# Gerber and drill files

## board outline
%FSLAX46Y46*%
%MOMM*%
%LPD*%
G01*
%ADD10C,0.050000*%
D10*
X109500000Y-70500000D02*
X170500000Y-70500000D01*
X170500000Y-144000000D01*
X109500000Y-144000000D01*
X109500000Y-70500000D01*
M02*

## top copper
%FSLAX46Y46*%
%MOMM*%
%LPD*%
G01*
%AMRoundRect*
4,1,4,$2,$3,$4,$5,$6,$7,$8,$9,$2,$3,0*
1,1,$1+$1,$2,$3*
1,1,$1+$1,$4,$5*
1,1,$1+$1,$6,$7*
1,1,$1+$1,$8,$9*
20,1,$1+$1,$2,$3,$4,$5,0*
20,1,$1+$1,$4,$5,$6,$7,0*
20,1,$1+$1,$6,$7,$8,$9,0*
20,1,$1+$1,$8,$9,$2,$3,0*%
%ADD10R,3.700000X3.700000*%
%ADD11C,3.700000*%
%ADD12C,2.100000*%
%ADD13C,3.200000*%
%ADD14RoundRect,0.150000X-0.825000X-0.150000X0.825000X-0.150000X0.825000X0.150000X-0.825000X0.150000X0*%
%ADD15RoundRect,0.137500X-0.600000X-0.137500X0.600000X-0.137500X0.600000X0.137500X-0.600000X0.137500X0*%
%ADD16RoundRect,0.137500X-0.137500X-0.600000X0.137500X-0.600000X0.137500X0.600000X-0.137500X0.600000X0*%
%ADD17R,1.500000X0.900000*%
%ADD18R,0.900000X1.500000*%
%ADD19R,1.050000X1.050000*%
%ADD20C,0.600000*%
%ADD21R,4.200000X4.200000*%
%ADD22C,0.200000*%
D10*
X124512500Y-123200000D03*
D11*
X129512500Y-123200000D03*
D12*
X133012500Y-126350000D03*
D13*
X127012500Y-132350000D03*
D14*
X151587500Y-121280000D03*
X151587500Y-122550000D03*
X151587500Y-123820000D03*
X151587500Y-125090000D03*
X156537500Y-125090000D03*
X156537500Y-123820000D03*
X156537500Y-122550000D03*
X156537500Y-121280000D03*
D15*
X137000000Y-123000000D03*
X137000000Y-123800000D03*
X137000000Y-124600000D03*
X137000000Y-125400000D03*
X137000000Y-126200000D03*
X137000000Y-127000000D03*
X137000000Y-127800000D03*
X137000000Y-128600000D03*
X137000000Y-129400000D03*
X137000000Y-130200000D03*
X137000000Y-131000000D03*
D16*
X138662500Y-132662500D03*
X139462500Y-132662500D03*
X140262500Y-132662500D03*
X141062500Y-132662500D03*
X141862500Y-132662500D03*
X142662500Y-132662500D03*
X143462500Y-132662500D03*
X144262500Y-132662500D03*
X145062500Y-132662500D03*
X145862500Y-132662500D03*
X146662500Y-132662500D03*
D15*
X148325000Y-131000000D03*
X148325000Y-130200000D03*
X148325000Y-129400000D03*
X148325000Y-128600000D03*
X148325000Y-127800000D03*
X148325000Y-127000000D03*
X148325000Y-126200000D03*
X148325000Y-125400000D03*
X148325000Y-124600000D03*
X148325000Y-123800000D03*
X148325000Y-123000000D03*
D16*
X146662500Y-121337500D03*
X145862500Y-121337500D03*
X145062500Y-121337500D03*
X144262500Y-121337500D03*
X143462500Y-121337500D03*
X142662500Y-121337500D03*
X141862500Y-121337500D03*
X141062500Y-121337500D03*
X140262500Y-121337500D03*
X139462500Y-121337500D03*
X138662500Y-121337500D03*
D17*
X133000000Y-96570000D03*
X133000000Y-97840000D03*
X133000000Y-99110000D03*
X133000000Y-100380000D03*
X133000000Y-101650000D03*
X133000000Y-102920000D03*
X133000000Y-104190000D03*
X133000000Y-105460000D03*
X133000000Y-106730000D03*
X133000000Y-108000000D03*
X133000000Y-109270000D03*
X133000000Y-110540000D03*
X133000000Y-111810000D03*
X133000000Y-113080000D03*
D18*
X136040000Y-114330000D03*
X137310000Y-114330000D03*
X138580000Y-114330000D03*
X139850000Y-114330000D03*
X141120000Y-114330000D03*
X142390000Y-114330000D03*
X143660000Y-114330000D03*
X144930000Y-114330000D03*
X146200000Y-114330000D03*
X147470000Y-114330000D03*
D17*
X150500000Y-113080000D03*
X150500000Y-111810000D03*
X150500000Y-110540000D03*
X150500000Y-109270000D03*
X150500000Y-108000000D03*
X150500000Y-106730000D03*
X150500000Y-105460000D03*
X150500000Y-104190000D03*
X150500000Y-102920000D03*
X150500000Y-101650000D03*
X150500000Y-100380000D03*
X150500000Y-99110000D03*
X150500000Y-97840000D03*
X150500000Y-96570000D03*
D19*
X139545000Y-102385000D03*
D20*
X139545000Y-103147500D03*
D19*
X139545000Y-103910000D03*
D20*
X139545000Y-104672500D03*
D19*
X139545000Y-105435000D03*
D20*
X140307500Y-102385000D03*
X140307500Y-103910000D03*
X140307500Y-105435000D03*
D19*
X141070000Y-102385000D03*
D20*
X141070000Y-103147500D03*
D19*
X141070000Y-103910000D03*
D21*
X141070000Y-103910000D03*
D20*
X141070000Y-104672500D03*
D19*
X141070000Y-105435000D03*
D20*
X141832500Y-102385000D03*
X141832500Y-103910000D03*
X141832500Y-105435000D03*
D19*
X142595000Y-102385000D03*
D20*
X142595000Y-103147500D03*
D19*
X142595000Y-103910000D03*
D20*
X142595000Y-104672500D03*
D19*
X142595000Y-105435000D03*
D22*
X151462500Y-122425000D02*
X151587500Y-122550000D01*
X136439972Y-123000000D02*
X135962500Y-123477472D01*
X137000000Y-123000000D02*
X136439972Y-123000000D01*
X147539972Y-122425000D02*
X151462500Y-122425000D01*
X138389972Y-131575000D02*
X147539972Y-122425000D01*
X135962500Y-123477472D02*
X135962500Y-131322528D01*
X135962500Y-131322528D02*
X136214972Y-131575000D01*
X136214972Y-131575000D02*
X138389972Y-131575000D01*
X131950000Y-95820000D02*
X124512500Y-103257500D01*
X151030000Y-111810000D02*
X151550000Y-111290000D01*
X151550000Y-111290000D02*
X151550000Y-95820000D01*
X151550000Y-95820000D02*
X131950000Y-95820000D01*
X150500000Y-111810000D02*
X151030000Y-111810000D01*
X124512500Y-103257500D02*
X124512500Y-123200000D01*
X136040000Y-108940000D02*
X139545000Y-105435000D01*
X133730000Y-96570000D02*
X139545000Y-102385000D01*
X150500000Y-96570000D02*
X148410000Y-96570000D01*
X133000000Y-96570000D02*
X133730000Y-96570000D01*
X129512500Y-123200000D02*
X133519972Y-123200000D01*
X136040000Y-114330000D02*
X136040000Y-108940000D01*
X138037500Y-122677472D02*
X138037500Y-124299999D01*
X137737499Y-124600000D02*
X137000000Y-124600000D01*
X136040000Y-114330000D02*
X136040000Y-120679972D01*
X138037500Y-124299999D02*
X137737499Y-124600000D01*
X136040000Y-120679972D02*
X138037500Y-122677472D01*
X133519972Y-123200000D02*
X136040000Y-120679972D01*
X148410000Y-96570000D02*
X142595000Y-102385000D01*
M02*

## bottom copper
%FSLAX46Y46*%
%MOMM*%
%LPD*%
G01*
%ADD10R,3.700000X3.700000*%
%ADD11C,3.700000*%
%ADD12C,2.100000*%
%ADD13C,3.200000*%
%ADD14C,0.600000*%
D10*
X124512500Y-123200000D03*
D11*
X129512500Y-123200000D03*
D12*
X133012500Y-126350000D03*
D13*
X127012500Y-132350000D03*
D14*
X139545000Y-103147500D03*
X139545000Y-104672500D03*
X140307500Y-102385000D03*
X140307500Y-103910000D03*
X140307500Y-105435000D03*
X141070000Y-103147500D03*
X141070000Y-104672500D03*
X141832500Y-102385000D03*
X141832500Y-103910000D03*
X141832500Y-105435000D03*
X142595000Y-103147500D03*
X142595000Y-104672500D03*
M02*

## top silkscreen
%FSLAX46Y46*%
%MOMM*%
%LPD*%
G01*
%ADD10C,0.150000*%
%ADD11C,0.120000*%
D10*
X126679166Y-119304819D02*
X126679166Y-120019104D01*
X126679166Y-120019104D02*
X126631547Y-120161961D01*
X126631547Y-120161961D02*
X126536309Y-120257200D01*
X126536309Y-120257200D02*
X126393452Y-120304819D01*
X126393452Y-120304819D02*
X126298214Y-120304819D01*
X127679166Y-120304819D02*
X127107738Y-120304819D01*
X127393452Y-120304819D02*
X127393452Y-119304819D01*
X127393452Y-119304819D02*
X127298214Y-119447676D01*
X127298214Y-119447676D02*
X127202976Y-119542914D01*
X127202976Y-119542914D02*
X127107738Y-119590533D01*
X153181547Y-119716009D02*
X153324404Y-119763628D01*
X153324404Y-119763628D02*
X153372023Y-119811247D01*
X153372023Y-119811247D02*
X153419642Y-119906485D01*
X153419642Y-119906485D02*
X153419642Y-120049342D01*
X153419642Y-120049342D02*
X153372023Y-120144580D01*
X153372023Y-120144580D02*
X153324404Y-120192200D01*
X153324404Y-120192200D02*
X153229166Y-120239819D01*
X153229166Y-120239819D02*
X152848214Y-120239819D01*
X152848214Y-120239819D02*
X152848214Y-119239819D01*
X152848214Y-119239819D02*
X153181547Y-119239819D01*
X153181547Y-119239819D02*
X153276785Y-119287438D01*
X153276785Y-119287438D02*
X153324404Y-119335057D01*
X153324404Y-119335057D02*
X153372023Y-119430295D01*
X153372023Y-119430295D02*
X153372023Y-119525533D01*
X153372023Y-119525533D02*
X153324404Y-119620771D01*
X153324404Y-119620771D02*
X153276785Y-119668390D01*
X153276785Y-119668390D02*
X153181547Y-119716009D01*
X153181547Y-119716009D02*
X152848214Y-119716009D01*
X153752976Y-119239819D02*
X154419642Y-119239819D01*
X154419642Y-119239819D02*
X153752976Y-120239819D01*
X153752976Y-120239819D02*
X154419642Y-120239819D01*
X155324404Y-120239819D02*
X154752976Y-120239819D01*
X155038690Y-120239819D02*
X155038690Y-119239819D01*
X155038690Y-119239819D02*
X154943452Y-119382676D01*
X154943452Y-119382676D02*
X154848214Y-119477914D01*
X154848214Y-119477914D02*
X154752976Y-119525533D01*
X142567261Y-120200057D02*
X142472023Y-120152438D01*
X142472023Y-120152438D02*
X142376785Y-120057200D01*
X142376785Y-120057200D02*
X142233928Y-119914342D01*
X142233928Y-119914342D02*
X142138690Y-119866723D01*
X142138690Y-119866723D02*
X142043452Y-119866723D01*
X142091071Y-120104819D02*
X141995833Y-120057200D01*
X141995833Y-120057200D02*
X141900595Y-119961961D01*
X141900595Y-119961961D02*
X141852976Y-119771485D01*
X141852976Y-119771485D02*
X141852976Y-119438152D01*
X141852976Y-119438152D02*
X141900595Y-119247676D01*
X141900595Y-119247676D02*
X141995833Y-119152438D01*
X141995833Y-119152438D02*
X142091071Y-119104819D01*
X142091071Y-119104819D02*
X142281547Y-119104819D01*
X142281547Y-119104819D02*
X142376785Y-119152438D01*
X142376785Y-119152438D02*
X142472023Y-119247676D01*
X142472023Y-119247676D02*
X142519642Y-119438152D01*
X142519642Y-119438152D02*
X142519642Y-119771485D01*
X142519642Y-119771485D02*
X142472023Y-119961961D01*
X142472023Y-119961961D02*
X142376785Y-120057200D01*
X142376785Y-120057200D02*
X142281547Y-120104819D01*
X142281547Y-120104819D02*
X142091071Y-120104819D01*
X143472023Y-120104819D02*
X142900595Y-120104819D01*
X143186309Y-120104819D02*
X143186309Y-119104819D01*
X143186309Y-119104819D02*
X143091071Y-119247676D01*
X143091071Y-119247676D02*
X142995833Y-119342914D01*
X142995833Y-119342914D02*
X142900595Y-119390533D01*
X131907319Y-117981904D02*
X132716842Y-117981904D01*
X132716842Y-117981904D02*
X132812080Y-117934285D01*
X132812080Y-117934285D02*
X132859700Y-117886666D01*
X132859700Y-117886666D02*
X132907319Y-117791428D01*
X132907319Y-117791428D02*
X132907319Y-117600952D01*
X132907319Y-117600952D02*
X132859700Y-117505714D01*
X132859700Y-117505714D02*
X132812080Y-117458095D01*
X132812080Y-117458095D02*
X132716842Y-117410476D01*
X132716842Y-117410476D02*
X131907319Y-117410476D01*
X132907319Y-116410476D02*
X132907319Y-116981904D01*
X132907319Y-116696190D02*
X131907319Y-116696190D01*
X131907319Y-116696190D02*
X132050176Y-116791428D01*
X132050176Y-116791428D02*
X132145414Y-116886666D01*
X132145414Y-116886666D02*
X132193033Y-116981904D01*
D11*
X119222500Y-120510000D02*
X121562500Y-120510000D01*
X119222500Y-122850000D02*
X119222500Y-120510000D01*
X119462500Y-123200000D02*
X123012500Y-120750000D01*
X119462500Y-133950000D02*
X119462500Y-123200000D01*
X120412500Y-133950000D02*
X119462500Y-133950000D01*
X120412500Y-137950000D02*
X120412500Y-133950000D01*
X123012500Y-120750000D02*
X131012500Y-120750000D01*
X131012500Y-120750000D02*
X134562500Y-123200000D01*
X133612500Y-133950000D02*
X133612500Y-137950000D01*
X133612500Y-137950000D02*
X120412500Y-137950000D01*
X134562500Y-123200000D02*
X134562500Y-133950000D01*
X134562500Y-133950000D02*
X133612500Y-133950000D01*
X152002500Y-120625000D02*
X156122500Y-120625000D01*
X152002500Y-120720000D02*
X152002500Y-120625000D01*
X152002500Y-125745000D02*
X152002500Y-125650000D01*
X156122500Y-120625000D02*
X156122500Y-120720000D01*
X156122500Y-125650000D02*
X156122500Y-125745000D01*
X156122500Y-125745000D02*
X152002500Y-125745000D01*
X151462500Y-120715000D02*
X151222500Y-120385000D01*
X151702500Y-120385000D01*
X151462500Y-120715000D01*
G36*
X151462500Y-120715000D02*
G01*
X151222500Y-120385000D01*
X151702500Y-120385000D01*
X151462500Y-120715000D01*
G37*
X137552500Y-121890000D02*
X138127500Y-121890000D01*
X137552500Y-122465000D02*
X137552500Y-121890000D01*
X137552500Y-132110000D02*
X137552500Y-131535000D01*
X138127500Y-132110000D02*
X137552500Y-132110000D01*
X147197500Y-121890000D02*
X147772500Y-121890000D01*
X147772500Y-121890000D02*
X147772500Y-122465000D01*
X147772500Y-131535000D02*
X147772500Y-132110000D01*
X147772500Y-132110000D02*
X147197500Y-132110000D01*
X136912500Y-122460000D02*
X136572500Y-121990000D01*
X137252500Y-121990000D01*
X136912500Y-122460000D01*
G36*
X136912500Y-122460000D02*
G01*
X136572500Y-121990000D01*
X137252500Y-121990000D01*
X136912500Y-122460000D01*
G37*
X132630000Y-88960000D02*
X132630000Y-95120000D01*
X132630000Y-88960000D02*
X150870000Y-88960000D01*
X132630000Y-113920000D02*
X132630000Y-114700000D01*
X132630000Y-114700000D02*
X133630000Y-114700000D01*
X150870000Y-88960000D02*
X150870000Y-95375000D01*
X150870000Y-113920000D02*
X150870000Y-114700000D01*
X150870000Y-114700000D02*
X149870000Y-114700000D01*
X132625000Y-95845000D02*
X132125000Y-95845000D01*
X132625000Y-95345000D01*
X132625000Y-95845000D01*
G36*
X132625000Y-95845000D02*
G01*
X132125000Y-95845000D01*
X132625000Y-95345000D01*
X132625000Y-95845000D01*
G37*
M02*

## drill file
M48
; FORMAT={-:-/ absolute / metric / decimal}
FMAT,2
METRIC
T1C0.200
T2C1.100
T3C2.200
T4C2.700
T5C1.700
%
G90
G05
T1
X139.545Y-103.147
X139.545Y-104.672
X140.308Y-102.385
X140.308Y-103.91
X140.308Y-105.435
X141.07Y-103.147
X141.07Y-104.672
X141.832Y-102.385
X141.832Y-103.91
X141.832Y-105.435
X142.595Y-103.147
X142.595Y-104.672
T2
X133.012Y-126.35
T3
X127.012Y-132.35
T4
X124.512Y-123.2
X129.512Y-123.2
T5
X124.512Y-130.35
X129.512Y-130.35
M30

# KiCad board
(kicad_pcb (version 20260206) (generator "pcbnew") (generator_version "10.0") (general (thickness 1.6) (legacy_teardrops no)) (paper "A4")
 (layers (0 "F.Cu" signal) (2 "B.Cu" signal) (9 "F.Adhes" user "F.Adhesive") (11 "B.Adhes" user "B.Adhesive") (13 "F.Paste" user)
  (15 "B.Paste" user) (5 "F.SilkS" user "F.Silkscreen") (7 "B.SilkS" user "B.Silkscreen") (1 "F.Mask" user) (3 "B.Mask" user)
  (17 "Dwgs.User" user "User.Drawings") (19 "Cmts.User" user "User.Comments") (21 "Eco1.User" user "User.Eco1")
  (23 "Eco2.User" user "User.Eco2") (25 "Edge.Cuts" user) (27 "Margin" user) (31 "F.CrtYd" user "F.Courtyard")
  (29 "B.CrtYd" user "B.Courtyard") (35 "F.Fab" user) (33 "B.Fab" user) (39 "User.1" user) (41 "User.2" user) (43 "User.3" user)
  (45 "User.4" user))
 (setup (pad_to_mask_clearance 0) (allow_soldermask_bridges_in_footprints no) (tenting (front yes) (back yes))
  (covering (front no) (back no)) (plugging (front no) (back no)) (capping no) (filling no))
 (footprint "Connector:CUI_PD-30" (layer "F.Cu") (at 124.5125 123.2)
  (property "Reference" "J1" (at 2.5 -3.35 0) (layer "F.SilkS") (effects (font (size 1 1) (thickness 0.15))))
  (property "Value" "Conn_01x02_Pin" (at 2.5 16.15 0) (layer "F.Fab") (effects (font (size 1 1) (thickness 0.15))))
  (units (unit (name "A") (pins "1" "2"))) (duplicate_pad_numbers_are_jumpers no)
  (fp_line (start -5.29 -2.69) (end -2.95 -2.69) (stroke (width 0.12) (type solid)) (layer "F.SilkS"))
  (fp_line (start -5.29 -0.35) (end -5.29 -2.69) (stroke (width 0.12) (type solid)) (layer "F.SilkS"))
  (fp_line (start -5.05 0) (end -1.5 -2.45) (stroke (width 0.12) (type solid)) (layer "F.SilkS"))
  (fp_line (start -5.05 10.75) (end -5.05 0) (stroke (width 0.12) (type solid)) (layer "F.SilkS"))
  (fp_line (start -4.1 10.75) (end -5.05 10.75) (stroke (width 0.12) (type solid)) (layer "F.SilkS"))
  (fp_line (start -4.1 14.75) (end -4.1 10.75) (stroke (width 0.12) (type solid)) (layer "F.SilkS"))
  (fp_line (start -1.5 -2.45) (end 6.5 -2.45) (stroke (width 0.12) (type solid)) (layer "F.SilkS"))
  (fp_line (start 6.5 -2.45) (end 10.05 0) (stroke (width 0.12) (type solid)) (layer "F.SilkS"))
  (fp_line (start 9.1 10.75) (end 9.1 14.75) (stroke (width 0.12) (type solid)) (layer "F.SilkS"))
  (fp_line (start 9.1 14.75) (end -4.1 14.75) (stroke (width 0.12) (type solid)) (layer "F.SilkS"))
  (fp_line (start 10.05 0) (end 10.05 10.75) (stroke (width 0.12) (type solid)) (layer "F.SilkS"))
  (fp_line (start 10.05 10.75) (end 9.1 10.75) (stroke (width 0.12) (type solid)) (layer "F.SilkS"))
  (pad "" np_thru_hole circle (at 0 7.15 180) (size 1.7 1.7) (drill 1.7) (layers "*.Cu" "*.Mask"))
  (pad "" np_thru_hole circle (at 5 7.15 180) (size 1.7 1.7) (drill 1.7) (layers "*.Cu" "*.Mask"))
  (pad "1" thru_hole rect (at 0 0 180) (size 3.7 3.7) (drill 2.7) (layers "*.Cu" "*.Mask") (remove_unused_layers no) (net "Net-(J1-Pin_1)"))
  (pad "2" thru_hole circle (at 5 0 180) (size 3.7 3.7) (drill 2.7) (layers "*.Cu" "*.Mask") (remove_unused_layers no) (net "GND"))
  (pad "3" thru_hole circle (at 8.5 3.15 180) (size 2.1 2.1) (drill 1.1) (layers "*.Cu" "*.Mask") (remove_unused_layers no))
  (pad "4" thru_hole circle (at 2.5 9.15 180) (size 3.2 3.2) (drill 2.2) (layers "*.Cu" "*.Mask") (remove_unused_layers no)))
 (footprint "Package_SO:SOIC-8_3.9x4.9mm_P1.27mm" (layer "F.Cu") (at 154.0625 123.185)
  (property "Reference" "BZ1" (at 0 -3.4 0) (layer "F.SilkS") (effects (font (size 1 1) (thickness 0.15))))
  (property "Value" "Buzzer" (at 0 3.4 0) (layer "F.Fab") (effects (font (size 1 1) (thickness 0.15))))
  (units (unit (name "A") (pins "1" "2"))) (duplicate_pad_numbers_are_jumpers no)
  (fp_line (start -2.06 -2.56) (end 2.06 -2.56) (stroke (width 0.12) (type solid)) (layer "F.SilkS"))
  (fp_line (start -2.06 -2.465) (end -2.06 -2.56) (stroke (width 0.12) (type solid)) (layer "F.SilkS"))
  (fp_line (start -2.06 2.56) (end -2.06 2.465) (stroke (width 0.12) (type solid)) (layer "F.SilkS"))
  (fp_line (start 2.06 -2.56) (end 2.06 -2.465) (stroke (width 0.12) (type solid)) (layer "F.SilkS"))
  (fp_line (start 2.06 2.465) (end 2.06 2.56) (stroke (width 0.12) (type solid)) (layer "F.SilkS"))
  (fp_line (start 2.06 2.56) (end -2.06 2.56) (stroke (width 0.12) (type solid)) (layer "F.SilkS"))
  (fp_poly (pts (xy -2.6 -2.47) (xy -2.84 -2.8) (xy -2.36 -2.8)) (stroke (width 0.12) (type solid)) (fill yes) (layer "F.SilkS"))
  (pad "1" smd roundrect (at -2.475 -1.905) (size 1.95 0.6) (layers "F.Cu" "F.Mask" "F.Paste") (roundrect_rratio 0.25) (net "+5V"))
  (pad "2" smd roundrect (at -2.475 -0.635) (size 1.95 0.6) (layers "F.Cu" "F.Mask" "F.Paste") (roundrect_rratio 0.25) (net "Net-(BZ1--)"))
  (pad "3" smd roundrect (at -2.475 0.635) (size 1.95 0.6) (layers "F.Cu" "F.Mask" "F.Paste") (roundrect_rratio 0.25))
  (pad "4" smd roundrect (at -2.475 1.905) (size 1.95 0.6) (layers "F.Cu" "F.Mask" "F.Paste") (roundrect_rratio 0.25))
  (pad "5" smd roundrect (at 2.475 1.905) (size 1.95 0.6) (layers "F.Cu" "F.Mask" "F.Paste") (roundrect_rratio 0.25))
  (pad "6" smd roundrect (at 2.475 0.635) (size 1.95 0.6) (layers "F.Cu" "F.Mask" "F.Paste") (roundrect_rratio 0.25))
  (pad "7" smd roundrect (at 2.475 -0.635) (size 1.95 0.6) (layers "F.Cu" "F.Mask" "F.Paste") (roundrect_rratio 0.25))
  (pad "8" smd roundrect (at 2.475 -1.905) (size 1.95 0.6) (layers "F.Cu" "F.Mask" "F.Paste") (roundrect_rratio 0.25)))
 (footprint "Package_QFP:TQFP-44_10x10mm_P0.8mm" (layer "F.Cu") (at 142.6625 127)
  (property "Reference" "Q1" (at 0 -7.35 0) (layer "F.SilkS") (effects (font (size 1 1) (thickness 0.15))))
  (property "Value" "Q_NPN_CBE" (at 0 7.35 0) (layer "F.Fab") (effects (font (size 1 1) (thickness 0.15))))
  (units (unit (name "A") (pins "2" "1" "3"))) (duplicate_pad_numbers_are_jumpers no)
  (fp_line (start -5.11 -5.11) (end -4.535 -5.11) (stroke (width 0.12) (type solid)) (layer "F.SilkS"))
  (fp_line (start -5.11 -4.535) (end -5.11 -5.11) (stroke (width 0.12) (type solid)) (layer "F.SilkS"))
  (fp_line (start -5.11 5.11) (end -5.11 4.535) (stroke (width 0.12) (type solid)) (layer "F.SilkS"))
  (fp_line (start -4.535 5.11) (end -5.11 5.11) (stroke (width 0.12) (type solid)) (layer "F.SilkS"))
  (fp_line (start 4.535 -5.11) (end 5.11 -5.11) (stroke (width 0.12) (type solid)) (layer "F.SilkS"))
  (fp_line (start 5.11 -5.11) (end 5.11 -4.535) (stroke (width 0.12) (type solid)) (layer "F.SilkS"))
  (fp_line (start 5.11 4.535) (end 5.11 5.11) (stroke (width 0.12) (type solid)) (layer "F.SilkS"))
  (fp_line (start 5.11 5.11) (end 4.535 5.11) (stroke (width 0.12) (type solid)) (layer "F.SilkS"))
  (fp_poly (pts (xy -5.75 -4.54) (xy -6.09 -5.01) (xy -5.41 -5.01)) (stroke (width 0.12) (type solid)) (fill yes) (layer "F.SilkS"))
  (pad "1" smd roundrect (at -5.6625 -4) (size 1.475 0.55) (layers "F.Cu" "F.Mask" "F.Paste") (roundrect_rratio 0.25) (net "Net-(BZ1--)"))
  (pad "2" smd roundrect (at -5.6625 -3.2) (size 1.475 0.55) (layers "F.Cu" "F.Mask" "F.Paste") (roundrect_rratio 0.25) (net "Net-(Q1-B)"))
  (pad "3" smd roundrect (at -5.6625 -2.4) (size 1.475 0.55) (layers "F.Cu" "F.Mask" "F.Paste") (roundrect_rratio 0.25) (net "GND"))
  (pad "4" smd roundrect (at -5.6625 -1.6) (size 1.475 0.55) (layers "F.Cu" "F.Mask" "F.Paste") (roundrect_rratio 0.25))
  (pad "5" smd roundrect (at -5.6625 -0.8) (size 1.475 0.55) (layers "F.Cu" "F.Mask" "F.Paste") (roundrect_rratio 0.25))
  (pad "6" smd roundrect (at -5.6625 0) (size 1.475 0.55) (layers "F.Cu" "F.Mask" "F.Paste") (roundrect_rratio 0.25))
  (pad "7" smd roundrect (at -5.6625 0.8) (size 1.475 0.55) (layers "F.Cu" "F.Mask" "F.Paste") (roundrect_rratio 0.25))
  (pad "8" smd roundrect (at -5.6625 1.6) (size 1.475 0.55) (layers "F.Cu" "F.Mask" "F.Paste") (roundrect_rratio 0.25))
  (pad "9" smd roundrect (at -5.6625 2.4) (size 1.475 0.55) (layers "F.Cu" "F.Mask" "F.Paste") (roundrect_rratio 0.25))
  (pad "10" smd roundrect (at -5.6625 3.2) (size 1.475 0.55) (layers "F.Cu" "F.Mask" "F.Paste") (roundrect_rratio 0.25))
  (pad "11" smd roundrect (at -5.6625 4) (size 1.475 0.55) (layers "F.Cu" "F.Mask" "F.Paste") (roundrect_rratio 0.25))
  (pad "12" smd roundrect (at -4 5.6625) (size 0.55 1.475) (layers "F.Cu" "F.Mask" "F.Paste") (roundrect_rratio 0.25))
  (pad "13" smd roundrect (at -3.2 5.6625) (size 0.55 1.475) (layers "F.Cu" "F.Mask" "F.Paste") (roundrect_rratio 0.25))
  (pad "14" smd roundrect (at -2.4 5.6625) (size 0.55 1.475) (layers "F.Cu" "F.Mask" "F.Paste") (roundrect_rratio 0.25))
  (pad "15" smd roundrect (at -1.6 5.6625) (size 0.55 1.475) (layers "F.Cu" "F.Mask" "F.Paste") (roundrect_rratio 0.25))
  (pad "16" smd roundrect (at -0.8 5.6625) (size 0.55 1.475) (layers "F.Cu" "F.Mask" "F.Paste") (roundrect_rratio 0.25))
  (pad "17" smd roundrect (at 0 5.6625) (size 0.55 1.475) (layers "F.Cu" "F.Mask" "F.Paste") (roundrect_rratio 0.25))
  (pad "18" smd roundrect (at 0.8 5.6625) (size 0.55 1.475) (layers "F.Cu" "F.Mask" "F.Paste") (roundrect_rratio 0.25))
  (pad "19" smd roundrect (at 1.6 5.6625) (size 0.55 1.475) (layers "F.Cu" "F.Mask" "F.Paste") (roundrect_rratio 0.25))
  (pad "20" smd roundrect (at 2.4 5.6625) (size 0.55 1.475) (layers "F.Cu" "F.Mask" "F.Paste") (roundrect_rratio 0.25))
  (pad "21" smd roundrect (at 3.2 5.6625) (size 0.55 1.475) (layers "F.Cu" "F.Mask" "F.Paste") (roundrect_rratio 0.25))
  (pad "22" smd roundrect (at 4 5.6625) (size 0.55 1.475) (layers "F.Cu" "F.Mask" "F.Paste") (roundrect_rratio 0.25))
  (pad "23" smd roundrect (at 5.6625 4) (size 1.475 0.55) (layers "F.Cu" "F.Mask" "F.Paste") (roundrect_rratio 0.25))
  (pad "24" smd roundrect (at 5.6625 3.2) (size 1.475 0.55) (layers "F.Cu" "F.Mask" "F.Paste") (roundrect_rratio 0.25))
  (pad "25" smd roundrect (at 5.6625 2.4) (size 1.475 0.55) (layers "F.Cu" "F.Mask" "F.Paste") (roundrect_rratio 0.25))
  (pad "26" smd roundrect (at 5.6625 1.6) (size 1.475 0.55) (layers "F.Cu" "F.Mask" "F.Paste") (roundrect_rratio 0.25))
  (pad "27" smd roundrect (at 5.6625 0.8) (size 1.475 0.55) (layers "F.Cu" "F.Mask" "F.Paste") (roundrect_rratio 0.25))
  (pad "28" smd roundrect (at 5.6625 0) (size 1.475 0.55) (layers "F.Cu" "F.Mask" "F.Paste") (roundrect_rratio 0.25))
  (pad "29" smd roundrect (at 5.6625 -0.8) (size 1.475 0.55) (layers "F.Cu" "F.Mask" "F.Paste") (roundrect_rratio 0.25))
  (pad "30" smd roundrect (at 5.6625 -1.6) (size 1.475 0.55) (layers "F.Cu" "F.Mask" "F.Paste") (roundrect_rratio 0.25))
  (pad "31" smd roundrect (at 5.6625 -2.4) (size 1.475 0.55) (layers "F.Cu" "F.Mask" "F.Paste") (roundrect_rratio 0.25))
  (pad "32" smd roundrect (at 5.6625 -3.2) (size 1.475 0.55) (layers "F.Cu" "F.Mask" "F.Paste") (roundrect_rratio 0.25))
  (pad "33" smd roundrect (at 5.6625 -4) (size 1.475 0.55) (layers "F.Cu" "F.Mask" "F.Paste") (roundrect_rratio 0.25))
  (pad "34" smd roundrect (at 4 -5.6625) (size 0.55 1.475) (layers "F.Cu" "F.Mask" "F.Paste") (roundrect_rratio 0.25))
  (pad "35" smd roundrect (at 3.2 -5.6625) (size 0.55 1.475) (layers "F.Cu" "F.Mask" "F.Paste") (roundrect_rratio 0.25))
  (pad "36" smd roundrect (at 2.4 -5.6625) (size 0.55 1.475) (layers "F.Cu" "F.Mask" "F.Paste") (roundrect_rratio 0.25))
  (pad "37" smd roundrect (at 1.6 -5.6625) (size 0.55 1.475) (layers "F.Cu" "F.Mask" "F.Paste") (roundrect_rratio 0.25))
  (pad "38" smd roundrect (at 0.8 -5.6625) (size 0.55 1.475) (layers "F.Cu" "F.Mask" "F.Paste") (roundrect_rratio 0.25))
  (pad "39" smd roundrect (at 0 -5.6625) (size 0.55 1.475) (layers "F.Cu" "F.Mask" "F.Paste") (roundrect_rratio 0.25))
  (pad "40" smd roundrect (at -0.8 -5.6625) (size 0.55 1.475) (layers "F.Cu" "F.Mask" "F.Paste") (roundrect_rratio 0.25))
  (pad "41" smd roundrect (at -1.6 -5.6625) (size 0.55 1.475) (layers "F.Cu" "F.Mask" "F.Paste") (roundrect_rratio 0.25))
  (pad "42" smd roundrect (at -2.4 -5.6625) (size 0.55 1.475) (layers "F.Cu" "F.Mask" "F.Paste") (roundrect_rratio 0.25))
  (pad "43" smd roundrect (at -3.2 -5.6625) (size 0.55 1.475) (layers "F.Cu" "F.Mask" "F.Paste") (roundrect_rratio 0.25))
  (pad "44" smd roundrect (at -4 -5.6625) (size 0.55 1.475) (layers "F.Cu" "F.Mask" "F.Paste") (roundrect_rratio 0.25)))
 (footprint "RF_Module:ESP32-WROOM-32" (layer "F.Cu") (at 141.75 104.82)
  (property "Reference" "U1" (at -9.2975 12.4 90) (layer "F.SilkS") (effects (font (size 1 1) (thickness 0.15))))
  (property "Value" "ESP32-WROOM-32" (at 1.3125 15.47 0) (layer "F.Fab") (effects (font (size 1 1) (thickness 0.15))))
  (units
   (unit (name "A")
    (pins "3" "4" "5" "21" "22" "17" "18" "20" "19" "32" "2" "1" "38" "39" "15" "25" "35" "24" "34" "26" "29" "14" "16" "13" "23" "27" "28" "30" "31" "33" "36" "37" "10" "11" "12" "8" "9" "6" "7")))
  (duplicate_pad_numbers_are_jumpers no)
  (fp_line (start -9.12 -15.86) (end -9.12 -9.7) (stroke (width 0.12) (type solid)) (layer "F.SilkS"))
  (fp_line (start -9.12 -15.86) (end 9.12 -15.86) (stroke (width 0.12) (type solid)) (layer "F.SilkS"))
  (fp_line (start -9.12 9.1) (end -9.12 9.88) (stroke (width 0.12) (type solid)) (layer "F.SilkS"))
  (fp_line (start -9.12 9.88) (end -8.12 9.88) (stroke (width 0.12) (type solid)) (layer "F.SilkS"))
  (fp_line (start 9.12 -15.86) (end 9.12 -9.445) (stroke (width 0.12) (type solid)) (layer "F.SilkS"))
  (fp_line (start 9.12 9.1) (end 9.12 9.88) (stroke (width 0.12) (type solid)) (layer "F.SilkS"))
  (fp_line (start 9.12 9.88) (end 8.12 9.88) (stroke (width 0.12) (type solid)) (layer "F.SilkS"))
  (fp_poly
   (pts (xy -9.125 -8.975) (xy -9.625 -8.975) (xy -9.125 -9.475) (xy -9.125 -8.975)) (stroke (width 0.12) (type solid)) (fill yes)
   (layer "F.SilkS"))
  (pad "1" smd rect (at -8.75 -8.25) (size 1.5 0.9) (layers "F.Cu" "F.Mask" "F.Paste") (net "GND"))
  (pad "2" smd rect (at -8.75 -6.98) (size 1.5 0.9) (layers "F.Cu" "F.Mask" "F.Paste") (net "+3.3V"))
  (pad "3" smd rect (at -8.75 -5.71) (size 1.5 0.9) (layers "F.Cu" "F.Mask" "F.Paste") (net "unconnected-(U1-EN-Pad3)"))
  (pad "4" smd rect (at -8.75 -4.44) (size 1.5 0.9) (layers "F.Cu" "F.Mask" "F.Paste") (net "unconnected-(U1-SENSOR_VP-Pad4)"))
  (pad "5" smd rect (at -8.75 -3.17) (size 1.5 0.9) (layers "F.Cu" "F.Mask" "F.Paste") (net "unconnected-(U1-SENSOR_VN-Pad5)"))
  (pad "6" smd rect (at -8.75 -1.9) (size 1.5 0.9) (layers "F.Cu" "F.Mask" "F.Paste") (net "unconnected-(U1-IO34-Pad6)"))
  (pad "7" smd rect (at -8.75 -0.63) (size 1.5 0.9) (layers "F.Cu" "F.Mask" "F.Paste") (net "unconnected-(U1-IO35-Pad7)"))
  (pad "8" smd rect (at -8.75 0.64) (size 1.5 0.9) (layers "F.Cu" "F.Mask" "F.Paste") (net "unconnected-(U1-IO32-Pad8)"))
  (pad "9" smd rect (at -8.75 1.91) (size 1.5 0.9) (layers "F.Cu" "F.Mask" "F.Paste") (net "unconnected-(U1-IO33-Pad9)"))
  (pad "10" smd rect (at -8.75 3.18) (size 1.5 0.9) (layers "F.Cu" "F.Mask" "F.Paste") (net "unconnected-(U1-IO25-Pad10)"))
  (pad "11" smd rect (at -8.75 4.45) (size 1.5 0.9) (layers "F.Cu" "F.Mask" "F.Paste") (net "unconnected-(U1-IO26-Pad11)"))
  (pad "12" smd rect (at -8.75 5.72) (size 1.5 0.9) (layers "F.Cu" "F.Mask" "F.Paste") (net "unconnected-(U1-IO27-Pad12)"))
  (pad "13" smd rect (at -8.75 6.99) (size 1.5 0.9) (layers "F.Cu" "F.Mask" "F.Paste") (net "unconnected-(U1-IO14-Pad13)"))
  (pad "14" smd rect (at -8.75 8.26) (size 1.5 0.9) (layers "F.Cu" "F.Mask" "F.Paste") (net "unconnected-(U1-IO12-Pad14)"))
  (pad "15" smd rect (at -5.71 9.51 90) (size 1.5 0.9) (layers "F.Cu" "F.Mask" "F.Paste") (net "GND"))
  (pad "16" smd rect (at -4.44 9.51 90) (size 1.5 0.9) (layers "F.Cu" "F.Mask" "F.Paste") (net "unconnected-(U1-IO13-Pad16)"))
  (pad "17" smd rect (at -3.17 9.51 90) (size 1.5 0.9) (layers "F.Cu" "F.Mask" "F.Paste") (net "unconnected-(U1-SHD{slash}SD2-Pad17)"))
  (pad "18" smd rect (at -1.9 9.51 90) (size 1.5 0.9) (layers "F.Cu" "F.Mask" "F.Paste") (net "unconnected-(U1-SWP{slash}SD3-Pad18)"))
  (pad "19" smd rect (at -0.63 9.51 90) (size 1.5 0.9) (layers "F.Cu" "F.Mask" "F.Paste") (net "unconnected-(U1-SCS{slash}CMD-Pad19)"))
  (pad "20" smd rect (at 0.64 9.51 90) (size 1.5 0.9) (layers "F.Cu" "F.Mask" "F.Paste") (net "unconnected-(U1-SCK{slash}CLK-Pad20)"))
  (pad "21" smd rect (at 1.91 9.51 90) (size 1.5 0.9) (layers "F.Cu" "F.Mask" "F.Paste") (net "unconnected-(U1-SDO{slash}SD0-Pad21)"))
  (pad "22" smd rect (at 3.18 9.51 90) (size 1.5 0.9) (layers "F.Cu" "F.Mask" "F.Paste") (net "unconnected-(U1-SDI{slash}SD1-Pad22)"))
  (pad "23" smd rect (at 4.45 9.51 90) (size 1.5 0.9) (layers "F.Cu" "F.Mask" "F.Paste") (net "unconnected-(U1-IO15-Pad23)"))
  (pad "24" smd rect (at 5.72 9.51 90) (size 1.5 0.9) (layers "F.Cu" "F.Mask" "F.Paste") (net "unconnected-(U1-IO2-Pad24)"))
  (pad "25" smd rect (at 8.75 8.26) (size 1.5 0.9) (layers "F.Cu" "F.Mask" "F.Paste") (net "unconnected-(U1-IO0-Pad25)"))
  (pad "26" smd rect (at 8.75 6.99) (size 1.5 0.9) (layers "F.Cu" "F.Mask" "F.Paste") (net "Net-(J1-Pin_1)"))
  (pad "27" smd rect (at 8.75 5.72) (size 1.5 0.9) (layers "F.Cu" "F.Mask" "F.Paste") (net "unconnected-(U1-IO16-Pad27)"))
  (pad "28" smd rect (at 8.75 4.45) (size 1.5 0.9) (layers "F.Cu" "F.Mask" "F.Paste") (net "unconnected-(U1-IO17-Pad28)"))
  (pad "29" smd rect (at 8.75 3.18) (size 1.5 0.9) (layers "F.Cu" "F.Mask" "F.Paste") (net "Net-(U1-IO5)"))
  (pad "30" smd rect (at 8.75 1.91) (size 1.5 0.9) (layers "F.Cu" "F.Mask" "F.Paste") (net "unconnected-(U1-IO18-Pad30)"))
  (pad "31" smd rect (at 8.75 0.64) (size 1.5 0.9) (layers "F.Cu" "F.Mask" "F.Paste") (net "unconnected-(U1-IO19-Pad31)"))
  (pad "32" smd rect (at 8.75 -0.63) (size 1.5 0.9) (layers "F.Cu" "F.Mask" "F.Paste") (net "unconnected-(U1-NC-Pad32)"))
  (pad "33" smd rect (at 8.75 -1.9) (size 1.5 0.9) (layers "F.Cu" "F.Mask" "F.Paste") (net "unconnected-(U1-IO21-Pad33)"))
  (pad "34" smd rect (at 8.75 -3.17) (size 1.5 0.9) (layers "F.Cu" "F.Mask" "F.Paste") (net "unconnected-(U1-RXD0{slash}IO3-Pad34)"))
  (pad "35" smd rect (at 8.75 -4.44) (size 1.5 0.9) (layers "F.Cu" "F.Mask" "F.Paste") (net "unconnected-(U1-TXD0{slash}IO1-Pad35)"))
  (pad "36" smd rect (at 8.75 -5.71) (size 1.5 0.9) (layers "F.Cu" "F.Mask" "F.Paste") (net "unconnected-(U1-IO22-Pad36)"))
  (pad "37" smd rect (at 8.75 -6.98) (size 1.5 0.9) (layers "F.Cu" "F.Mask" "F.Paste") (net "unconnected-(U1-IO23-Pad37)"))
  (pad "38" smd rect (at 8.75 -8.25) (size 1.5 0.9) (layers "F.Cu" "F.Mask" "F.Paste") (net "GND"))
  (pad "39" smd rect (at -2.205 -2.435) (size 1.05 1.05) (layers "F.Cu" "F.Paste") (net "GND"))
  (pad "39" thru_hole circle (at -2.205 -1.6725) (size 0.6 0.6) (drill 0.2) (layers "*.Cu" "F.Mask") (remove_unused_layers no) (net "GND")
   (zone_connect 2))
  (pad "39" smd rect (at -2.205 -0.91) (size 1.05 1.05) (layers "F.Cu" "F.Paste") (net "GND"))
  (pad "39" thru_hole circle (at -2.205 -0.1475) (size 0.6 0.6) (drill 0.2) (layers "*.Cu" "F.Mask") (remove_unused_layers no) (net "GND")
   (zone_connect 2))
  (pad "39" smd rect (at -2.205 0.615) (size 1.05 1.05) (layers "F.Cu" "F.Paste") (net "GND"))
  (pad "39" thru_hole circle (at -1.4425 -2.435) (size 0.6 0.6) (drill 0.2) (layers "*.Cu" "F.Mask") (remove_unused_layers no) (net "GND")
   (zone_connect 2))
  (pad "39" thru_hole circle (at -1.4425 -0.91) (size 0.6 0.6) (drill 0.2) (layers "*.Cu" "F.Mask") (remove_unused_layers no) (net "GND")
   (zone_connect 2))
  (pad "39" thru_hole circle (at -1.4425 0.615) (size 0.6 0.6) (drill 0.2) (layers "*.Cu" "F.Mask") (remove_unused_layers no) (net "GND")
   (zone_connect 2))
  (pad "39" smd rect (at -0.68 -2.435) (size 1.05 1.05) (layers "F.Cu" "F.Paste") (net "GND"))
  (pad "39" thru_hole circle (at -0.68 -1.6725) (size 0.6 0.6) (drill 0.2) (layers "*.Cu" "F.Mask") (remove_unused_layers no) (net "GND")
   (zone_connect 2))
  (pad "39" smd rect (at -0.68 -0.91) (size 1.05 1.05) (layers "F.Cu" "F.Paste") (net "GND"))
  (pad "39" smd rect (at -0.68 -0.91) (size 4.2 4.2) (layers "F.Cu" "F.Mask") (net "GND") (zone_connect 2))
  (pad "39" thru_hole circle (at -0.68 -0.1475) (size 0.6 0.6) (drill 0.2) (layers "*.Cu" "F.Mask") (remove_unused_layers no) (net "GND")
   (zone_connect 2))
  (pad "39" smd rect (at -0.68 0.615) (size 1.05 1.05) (layers "F.Cu" "F.Paste") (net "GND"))
  (pad "39" thru_hole circle (at 0.0825 -2.435) (size 0.6 0.6) (drill 0.2) (layers "*.Cu" "F.Mask") (remove_unused_layers no) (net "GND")
   (zone_connect 2))
  (pad "39" thru_hole circle (at 0.0825 -0.91) (size 0.6 0.6) (drill 0.2) (layers "*.Cu" "F.Mask") (remove_unused_layers no) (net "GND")
   (zone_connect 2))
  (pad "39" thru_hole circle (at 0.0825 0.615) (size 0.6 0.6) (drill 0.2) (layers "*.Cu" "F.Mask") (remove_unused_layers no) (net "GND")
   (zone_connect 2))
  (pad "39" smd rect (at 0.845 -2.435) (size 1.05 1.05) (layers "F.Cu" "F.Paste") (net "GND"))
  (pad "39" thru_hole circle (at 0.845 -1.6725) (size 0.6 0.6) (drill 0.2) (layers "*.Cu" "F.Mask") (remove_unused_layers no) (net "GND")
   (zone_connect 2))
  (pad "39" smd rect (at 0.845 -0.91) (size 1.05 1.05) (layers "F.Cu" "F.Paste") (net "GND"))
  (pad "39" thru_hole circle (at 0.845 -0.1475) (size 0.6 0.6) (drill 0.2) (layers "*.Cu" "F.Mask") (remove_unused_layers no) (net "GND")
   (zone_connect 2))
  (pad "39" smd rect (at 0.845 0.615) (size 1.05 1.05) (layers "F.Cu" "F.Paste") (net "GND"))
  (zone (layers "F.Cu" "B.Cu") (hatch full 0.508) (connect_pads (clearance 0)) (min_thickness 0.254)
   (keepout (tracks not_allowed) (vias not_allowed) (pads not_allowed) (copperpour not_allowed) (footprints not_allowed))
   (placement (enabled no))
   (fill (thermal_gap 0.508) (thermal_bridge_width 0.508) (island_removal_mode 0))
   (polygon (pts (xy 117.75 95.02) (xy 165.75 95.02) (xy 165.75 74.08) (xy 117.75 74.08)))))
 (gr_rect (start 109.5 70.5) (end 170.5 144) (stroke (width 0.05) (type default)) (fill no) (layer "Edge.Cuts"))
 (segment (start 151.4625 122.425) (end 151.5875 122.55) (width 0.2) (layer "F.Cu") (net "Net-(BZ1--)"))
 (segment (start 136.439972 123) (end 135.9625 123.477472) (width 0.2) (layer "F.Cu") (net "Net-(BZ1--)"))
 (segment (start 137 123) (end 136.439972 123) (width 0.2) (layer "F.Cu") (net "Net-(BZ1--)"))
 (segment (start 147.539972 122.425) (end 151.4625 122.425) (width 0.2) (layer "F.Cu") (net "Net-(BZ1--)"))
 (segment (start 138.389972 131.575) (end 147.539972 122.425) (width 0.2) (layer "F.Cu") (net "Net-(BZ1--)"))
 (segment (start 135.9625 123.477472) (end 135.9625 131.322528) (width 0.2) (layer "F.Cu") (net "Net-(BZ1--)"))
 (segment (start 135.9625 131.322528) (end 136.214972 131.575) (width 0.2) (layer "F.Cu") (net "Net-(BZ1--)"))
 (segment (start 136.214972 131.575) (end 138.389972 131.575) (width 0.2) (layer "F.Cu") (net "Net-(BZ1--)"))
 (segment (start 131.95 95.82) (end 124.5125 103.2575) (width 0.2) (layer "F.Cu") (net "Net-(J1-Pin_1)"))
 (segment (start 151.03 111.81) (end 151.55 111.29) (width 0.2) (layer "F.Cu") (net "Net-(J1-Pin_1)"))
 (segment (start 151.55 111.29) (end 151.55 95.82) (width 0.2) (layer "F.Cu") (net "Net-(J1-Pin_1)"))
 (segment (start 151.55 95.82) (end 131.95 95.82) (width 0.2) (layer "F.Cu") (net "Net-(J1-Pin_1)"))
 (segment (start 150.5 111.81) (end 151.03 111.81) (width 0.2) (layer "F.Cu") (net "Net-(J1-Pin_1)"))
 (segment (start 124.5125 103.2575) (end 124.5125 123.2) (width 0.2) (layer "F.Cu") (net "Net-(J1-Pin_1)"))
 (segment (start 136.04 108.94) (end 139.545 105.435) (width 0.2) (layer "F.Cu") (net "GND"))
 (segment (start 133.73 96.57) (end 139.545 102.385) (width 0.2) (layer "F.Cu") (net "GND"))
 (segment (start 150.5 96.57) (end 148.41 96.57) (width 0.2) (layer "F.Cu") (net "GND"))
 (segment (start 133 96.57) (end 133.73 96.57) (width 0.2) (layer "F.Cu") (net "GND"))
 (segment (start 129.5125 123.2) (end 133.519972 123.2) (width 0.2) (layer "F.Cu") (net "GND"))
 (segment (start 136.04 114.33) (end 136.04 108.94) (width 0.2) (layer "F.Cu") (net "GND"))
 (segment (start 138.0375 122.677472) (end 138.0375 124.299999) (width 0.2) (layer "F.Cu") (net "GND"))
 (segment (start 137.737499 124.6) (end 137 124.6) (width 0.2) (layer "F.Cu") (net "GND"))
 (segment (start 136.04 114.33) (end 136.04 120.679972) (width 0.2) (layer "F.Cu") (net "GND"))
 (segment (start 138.0375 124.299999) (end 137.737499 124.6) (width 0.2) (layer "F.Cu") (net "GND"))
 (segment (start 136.04 120.679972) (end 138.0375 122.677472) (width 0.2) (layer "F.Cu") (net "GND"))
 (segment (start 133.519972 123.2) (end 136.04 120.679972) (width 0.2) (layer "F.Cu") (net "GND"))
 (segment (start 148.41 96.57) (end 142.595 102.385) (width 0.2) (layer "F.Cu") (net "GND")))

